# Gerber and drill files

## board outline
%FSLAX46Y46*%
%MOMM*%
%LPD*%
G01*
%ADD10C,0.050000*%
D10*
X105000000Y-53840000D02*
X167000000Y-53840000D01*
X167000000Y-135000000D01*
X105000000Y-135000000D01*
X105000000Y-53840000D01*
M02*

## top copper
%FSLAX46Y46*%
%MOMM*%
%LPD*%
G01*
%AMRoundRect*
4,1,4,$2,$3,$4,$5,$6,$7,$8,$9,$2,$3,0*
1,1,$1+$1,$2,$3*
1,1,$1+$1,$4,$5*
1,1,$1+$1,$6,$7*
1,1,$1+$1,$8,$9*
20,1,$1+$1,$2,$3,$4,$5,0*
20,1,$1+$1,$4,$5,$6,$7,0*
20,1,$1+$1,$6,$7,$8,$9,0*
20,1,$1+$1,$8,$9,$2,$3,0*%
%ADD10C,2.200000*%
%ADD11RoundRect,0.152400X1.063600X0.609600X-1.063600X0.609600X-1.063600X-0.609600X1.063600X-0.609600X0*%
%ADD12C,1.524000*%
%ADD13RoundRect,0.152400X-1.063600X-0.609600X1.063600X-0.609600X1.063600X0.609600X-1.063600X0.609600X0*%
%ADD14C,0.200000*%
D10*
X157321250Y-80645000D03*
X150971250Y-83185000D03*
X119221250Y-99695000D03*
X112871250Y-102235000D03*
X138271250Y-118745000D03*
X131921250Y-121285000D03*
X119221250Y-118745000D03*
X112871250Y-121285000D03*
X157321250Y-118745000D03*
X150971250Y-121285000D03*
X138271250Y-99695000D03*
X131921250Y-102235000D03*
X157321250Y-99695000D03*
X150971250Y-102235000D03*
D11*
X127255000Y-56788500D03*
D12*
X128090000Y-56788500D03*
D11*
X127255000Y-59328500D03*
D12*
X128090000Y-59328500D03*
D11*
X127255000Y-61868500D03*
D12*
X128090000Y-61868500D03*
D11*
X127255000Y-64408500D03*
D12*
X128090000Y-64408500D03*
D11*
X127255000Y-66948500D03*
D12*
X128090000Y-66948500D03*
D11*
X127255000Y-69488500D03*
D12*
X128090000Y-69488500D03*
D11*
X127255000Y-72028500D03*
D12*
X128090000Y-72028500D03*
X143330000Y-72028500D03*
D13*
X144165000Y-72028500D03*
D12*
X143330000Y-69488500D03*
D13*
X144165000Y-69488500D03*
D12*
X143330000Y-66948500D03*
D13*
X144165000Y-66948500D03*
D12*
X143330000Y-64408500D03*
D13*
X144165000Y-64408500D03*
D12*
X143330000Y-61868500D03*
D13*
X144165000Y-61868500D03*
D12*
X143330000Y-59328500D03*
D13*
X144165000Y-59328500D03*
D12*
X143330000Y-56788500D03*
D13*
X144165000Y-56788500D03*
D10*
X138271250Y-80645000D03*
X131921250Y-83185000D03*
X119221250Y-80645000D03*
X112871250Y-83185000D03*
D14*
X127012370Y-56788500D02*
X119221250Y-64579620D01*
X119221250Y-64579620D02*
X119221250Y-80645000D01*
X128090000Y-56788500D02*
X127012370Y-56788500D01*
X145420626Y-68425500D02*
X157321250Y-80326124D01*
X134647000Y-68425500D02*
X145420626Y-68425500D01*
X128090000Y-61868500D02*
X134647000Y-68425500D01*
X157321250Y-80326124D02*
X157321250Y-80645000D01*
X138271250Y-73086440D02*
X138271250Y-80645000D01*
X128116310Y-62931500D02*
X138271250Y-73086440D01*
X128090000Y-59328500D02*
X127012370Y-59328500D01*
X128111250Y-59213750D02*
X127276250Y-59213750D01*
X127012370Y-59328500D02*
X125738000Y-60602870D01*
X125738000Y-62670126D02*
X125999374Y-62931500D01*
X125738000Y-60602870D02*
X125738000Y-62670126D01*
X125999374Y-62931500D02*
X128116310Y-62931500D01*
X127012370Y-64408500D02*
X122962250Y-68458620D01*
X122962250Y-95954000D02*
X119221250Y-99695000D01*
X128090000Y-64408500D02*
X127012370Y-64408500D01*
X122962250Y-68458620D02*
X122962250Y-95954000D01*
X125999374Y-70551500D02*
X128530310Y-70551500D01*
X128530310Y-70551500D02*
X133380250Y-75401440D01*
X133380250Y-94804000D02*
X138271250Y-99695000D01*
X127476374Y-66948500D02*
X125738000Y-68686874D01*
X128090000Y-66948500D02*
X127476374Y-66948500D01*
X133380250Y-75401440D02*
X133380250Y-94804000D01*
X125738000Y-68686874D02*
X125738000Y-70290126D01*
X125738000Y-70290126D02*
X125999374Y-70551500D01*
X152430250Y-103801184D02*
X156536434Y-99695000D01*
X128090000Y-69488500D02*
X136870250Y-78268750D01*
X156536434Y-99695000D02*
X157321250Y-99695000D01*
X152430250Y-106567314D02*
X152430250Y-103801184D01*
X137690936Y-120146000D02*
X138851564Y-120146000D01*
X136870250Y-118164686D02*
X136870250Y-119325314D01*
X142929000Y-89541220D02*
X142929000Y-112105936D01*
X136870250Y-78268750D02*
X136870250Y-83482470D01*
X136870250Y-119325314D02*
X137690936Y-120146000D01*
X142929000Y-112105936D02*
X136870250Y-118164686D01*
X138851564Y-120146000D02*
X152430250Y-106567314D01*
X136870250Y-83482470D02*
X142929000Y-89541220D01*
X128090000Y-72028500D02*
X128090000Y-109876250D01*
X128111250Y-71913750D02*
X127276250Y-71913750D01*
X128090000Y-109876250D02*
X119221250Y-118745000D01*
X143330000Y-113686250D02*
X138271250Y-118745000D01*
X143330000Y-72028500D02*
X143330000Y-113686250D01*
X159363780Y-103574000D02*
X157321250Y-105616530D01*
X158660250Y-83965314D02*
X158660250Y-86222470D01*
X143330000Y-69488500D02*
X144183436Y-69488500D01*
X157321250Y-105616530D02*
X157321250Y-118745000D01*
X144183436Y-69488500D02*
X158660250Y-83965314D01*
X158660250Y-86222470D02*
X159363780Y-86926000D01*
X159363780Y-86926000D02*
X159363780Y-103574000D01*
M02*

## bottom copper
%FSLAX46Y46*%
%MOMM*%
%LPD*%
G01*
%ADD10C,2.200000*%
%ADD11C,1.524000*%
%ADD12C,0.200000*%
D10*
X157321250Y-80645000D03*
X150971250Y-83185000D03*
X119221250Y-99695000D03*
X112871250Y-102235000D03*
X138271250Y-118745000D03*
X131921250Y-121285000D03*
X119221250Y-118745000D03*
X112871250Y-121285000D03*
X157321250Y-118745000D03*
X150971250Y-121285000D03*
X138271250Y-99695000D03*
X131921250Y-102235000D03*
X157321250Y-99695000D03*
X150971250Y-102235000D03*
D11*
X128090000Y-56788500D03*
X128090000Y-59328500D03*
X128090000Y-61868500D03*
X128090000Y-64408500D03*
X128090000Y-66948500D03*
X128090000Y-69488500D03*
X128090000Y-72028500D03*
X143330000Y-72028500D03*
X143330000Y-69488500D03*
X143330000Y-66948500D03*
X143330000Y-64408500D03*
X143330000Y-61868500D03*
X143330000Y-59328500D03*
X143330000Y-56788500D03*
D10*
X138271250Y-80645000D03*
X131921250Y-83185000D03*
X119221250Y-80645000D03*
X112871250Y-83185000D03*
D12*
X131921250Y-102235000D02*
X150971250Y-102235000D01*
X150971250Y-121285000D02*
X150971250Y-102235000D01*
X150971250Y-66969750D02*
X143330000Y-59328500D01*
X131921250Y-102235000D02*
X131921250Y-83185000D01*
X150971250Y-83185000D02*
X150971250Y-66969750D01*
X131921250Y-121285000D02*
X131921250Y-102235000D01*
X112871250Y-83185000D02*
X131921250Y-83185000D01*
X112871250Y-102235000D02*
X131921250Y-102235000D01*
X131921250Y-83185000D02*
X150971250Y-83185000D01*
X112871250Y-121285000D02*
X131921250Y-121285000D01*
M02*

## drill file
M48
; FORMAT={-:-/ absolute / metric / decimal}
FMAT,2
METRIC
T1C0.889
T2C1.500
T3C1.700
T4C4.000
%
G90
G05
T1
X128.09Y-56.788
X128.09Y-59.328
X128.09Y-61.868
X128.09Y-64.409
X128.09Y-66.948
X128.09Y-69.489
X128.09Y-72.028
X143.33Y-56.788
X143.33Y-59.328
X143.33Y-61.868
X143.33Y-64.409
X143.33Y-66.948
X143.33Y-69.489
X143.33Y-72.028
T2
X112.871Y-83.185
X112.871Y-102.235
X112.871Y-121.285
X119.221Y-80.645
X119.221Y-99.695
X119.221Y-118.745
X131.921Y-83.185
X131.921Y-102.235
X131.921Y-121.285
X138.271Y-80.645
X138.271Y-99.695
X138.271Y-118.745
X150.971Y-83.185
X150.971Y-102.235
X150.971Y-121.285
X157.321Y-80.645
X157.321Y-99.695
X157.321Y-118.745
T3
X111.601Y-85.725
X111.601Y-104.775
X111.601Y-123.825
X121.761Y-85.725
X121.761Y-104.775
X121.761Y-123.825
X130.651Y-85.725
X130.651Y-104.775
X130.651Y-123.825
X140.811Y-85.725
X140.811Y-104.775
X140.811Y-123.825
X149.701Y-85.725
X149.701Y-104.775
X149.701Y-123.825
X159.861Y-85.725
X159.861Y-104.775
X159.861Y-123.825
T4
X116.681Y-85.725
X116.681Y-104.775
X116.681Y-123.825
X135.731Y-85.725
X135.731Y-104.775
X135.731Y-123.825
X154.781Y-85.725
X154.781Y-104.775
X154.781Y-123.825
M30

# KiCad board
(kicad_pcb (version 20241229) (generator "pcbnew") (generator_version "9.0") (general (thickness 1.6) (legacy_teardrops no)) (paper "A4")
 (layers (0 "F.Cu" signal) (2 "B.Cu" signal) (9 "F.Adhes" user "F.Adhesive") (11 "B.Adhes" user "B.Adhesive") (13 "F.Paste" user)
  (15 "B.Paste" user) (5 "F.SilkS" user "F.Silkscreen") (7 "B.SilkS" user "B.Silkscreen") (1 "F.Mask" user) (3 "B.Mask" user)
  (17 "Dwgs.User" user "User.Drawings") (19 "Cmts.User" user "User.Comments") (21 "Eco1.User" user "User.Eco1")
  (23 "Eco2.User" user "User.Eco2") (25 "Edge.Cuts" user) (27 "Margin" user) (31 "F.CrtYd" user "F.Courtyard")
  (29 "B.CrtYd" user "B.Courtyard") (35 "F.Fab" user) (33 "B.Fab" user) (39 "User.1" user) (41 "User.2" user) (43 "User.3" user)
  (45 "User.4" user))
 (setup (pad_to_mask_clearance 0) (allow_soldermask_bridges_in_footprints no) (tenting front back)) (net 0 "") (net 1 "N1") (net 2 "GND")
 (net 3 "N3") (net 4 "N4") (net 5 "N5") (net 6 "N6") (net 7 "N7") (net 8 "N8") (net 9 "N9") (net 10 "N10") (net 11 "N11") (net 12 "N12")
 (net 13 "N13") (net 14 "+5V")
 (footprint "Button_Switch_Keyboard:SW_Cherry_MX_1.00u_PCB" (layer "F.Cu") (at 157.32125 80.645)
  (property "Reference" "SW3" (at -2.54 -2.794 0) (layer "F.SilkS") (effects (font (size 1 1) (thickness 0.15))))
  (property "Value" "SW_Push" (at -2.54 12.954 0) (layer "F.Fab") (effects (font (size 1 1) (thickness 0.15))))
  (pad "" np_thru_hole circle (at -7.62 5.08) (size 1.7 1.7) (drill 1.7) (layers "*.Cu" "*.Mask"))
  (pad "" np_thru_hole circle (at -2.54 5.08) (size 4 4) (drill 4) (layers "*.Cu" "*.Mask"))
  (pad "" np_thru_hole circle (at 2.54 5.08) (size 1.7 1.7) (drill 1.7) (layers "*.Cu" "*.Mask"))
  (pad "1" thru_hole circle (at 0 0) (size 2.2 2.2) (drill 1.5) (layers "*.Cu" "*.Mask") (remove_unused_layers no) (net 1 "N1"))
  (pad "2" thru_hole circle (at -6.35 2.54) (size 2.2 2.2) (drill 1.5) (layers "*.Cu" "*.Mask") (remove_unused_layers no) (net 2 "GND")))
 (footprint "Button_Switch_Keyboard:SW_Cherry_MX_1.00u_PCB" (layer "F.Cu") (at 119.22125 99.695)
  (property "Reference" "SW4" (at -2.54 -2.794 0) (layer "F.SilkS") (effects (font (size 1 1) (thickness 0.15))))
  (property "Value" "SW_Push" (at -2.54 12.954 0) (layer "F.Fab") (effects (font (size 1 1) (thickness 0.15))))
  (pad "" np_thru_hole circle (at -7.62 5.08) (size 1.7 1.7) (drill 1.7) (layers "*.Cu" "*.Mask"))
  (pad "" np_thru_hole circle (at -2.54 5.08) (size 4 4) (drill 4) (layers "*.Cu" "*.Mask"))
  (pad "" np_thru_hole circle (at 2.54 5.08) (size 1.7 1.7) (drill 1.7) (layers "*.Cu" "*.Mask"))
  (pad "1" thru_hole circle (at 0 0) (size 2.2 2.2) (drill 1.5) (layers "*.Cu" "*.Mask") (remove_unused_layers no) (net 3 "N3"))
  (pad "2" thru_hole circle (at -6.35 2.54) (size 2.2 2.2) (drill 1.5) (layers "*.Cu" "*.Mask") (remove_unused_layers no) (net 2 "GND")))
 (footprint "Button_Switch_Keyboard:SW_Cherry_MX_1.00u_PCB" (layer "F.Cu") (at 138.27125 118.745)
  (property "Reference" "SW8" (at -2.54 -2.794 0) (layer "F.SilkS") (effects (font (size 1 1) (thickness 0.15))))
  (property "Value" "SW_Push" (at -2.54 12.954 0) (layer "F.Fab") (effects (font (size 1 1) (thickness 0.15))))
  (pad "" np_thru_hole circle (at -7.62 5.08) (size 1.7 1.7) (drill 1.7) (layers "*.Cu" "*.Mask"))
  (pad "" np_thru_hole circle (at -2.54 5.08) (size 4 4) (drill 4) (layers "*.Cu" "*.Mask"))
  (pad "" np_thru_hole circle (at 2.54 5.08) (size 1.7 1.7) (drill 1.7) (layers "*.Cu" "*.Mask"))
  (pad "1" thru_hole circle (at 0 0) (size 2.2 2.2) (drill 1.5) (layers "*.Cu" "*.Mask") (remove_unused_layers no) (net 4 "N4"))
  (pad "2" thru_hole circle (at -6.35 2.54) (size 2.2 2.2) (drill 1.5) (layers "*.Cu" "*.Mask") (remove_unused_layers no) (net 2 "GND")))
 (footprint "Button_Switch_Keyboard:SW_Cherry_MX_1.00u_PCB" (layer "F.Cu") (at 119.22125 118.745)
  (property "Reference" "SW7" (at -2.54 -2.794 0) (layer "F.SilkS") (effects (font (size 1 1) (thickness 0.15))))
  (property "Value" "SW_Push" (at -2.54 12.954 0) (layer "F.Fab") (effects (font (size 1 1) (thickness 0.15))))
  (pad "" np_thru_hole circle (at -7.62 5.08) (size 1.7 1.7) (drill 1.7) (layers "*.Cu" "*.Mask"))
  (pad "" np_thru_hole circle (at -2.54 5.08) (size 4 4) (drill 4) (layers "*.Cu" "*.Mask"))
  (pad "" np_thru_hole circle (at 2.54 5.08) (size 1.7 1.7) (drill 1.7) (layers "*.Cu" "*.Mask"))
  (pad "1" thru_hole circle (at 0 0) (size 2.2 2.2) (drill 1.5) (layers "*.Cu" "*.Mask") (remove_unused_layers no) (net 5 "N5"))
  (pad "2" thru_hole circle (at -6.35 2.54) (size 2.2 2.2) (drill 1.5) (layers "*.Cu" "*.Mask") (remove_unused_layers no) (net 2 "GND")))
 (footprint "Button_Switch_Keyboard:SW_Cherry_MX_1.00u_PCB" (layer "F.Cu") (at 157.32125 118.745)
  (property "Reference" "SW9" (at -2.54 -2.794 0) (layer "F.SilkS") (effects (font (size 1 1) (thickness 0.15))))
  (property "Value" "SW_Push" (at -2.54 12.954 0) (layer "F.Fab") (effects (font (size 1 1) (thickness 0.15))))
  (pad "" np_thru_hole circle (at -7.62 5.08) (size 1.7 1.7) (drill 1.7) (layers "*.Cu" "*.Mask"))
  (pad "" np_thru_hole circle (at -2.54 5.08) (size 4 4) (drill 4) (layers "*.Cu" "*.Mask"))
  (pad "" np_thru_hole circle (at 2.54 5.08) (size 1.7 1.7) (drill 1.7) (layers "*.Cu" "*.Mask"))
  (pad "1" thru_hole circle (at 0 0) (size 2.2 2.2) (drill 1.5) (layers "*.Cu" "*.Mask") (remove_unused_layers no) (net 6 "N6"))
  (pad "2" thru_hole circle (at -6.35 2.54) (size 2.2 2.2) (drill 1.5) (layers "*.Cu" "*.Mask") (remove_unused_layers no) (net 2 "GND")))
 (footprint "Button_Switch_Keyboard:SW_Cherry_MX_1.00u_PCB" (layer "F.Cu") (at 138.27125 99.695)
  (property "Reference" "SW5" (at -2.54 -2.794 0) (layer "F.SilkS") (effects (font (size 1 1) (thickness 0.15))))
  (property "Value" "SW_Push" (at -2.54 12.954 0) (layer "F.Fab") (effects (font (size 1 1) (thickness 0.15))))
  (pad "" np_thru_hole circle (at -7.62 5.08) (size 1.7 1.7) (drill 1.7) (layers "*.Cu" "*.Mask"))
  (pad "" np_thru_hole circle (at -2.54 5.08) (size 4 4) (drill 4) (layers "*.Cu" "*.Mask"))
  (pad "" np_thru_hole circle (at 2.54 5.08) (size 1.7 1.7) (drill 1.7) (layers "*.Cu" "*.Mask"))
  (pad "1" thru_hole circle (at 0 0) (size 2.2 2.2) (drill 1.5) (layers "*.Cu" "*.Mask") (remove_unused_layers no) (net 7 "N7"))
  (pad "2" thru_hole circle (at -6.35 2.54) (size 2.2 2.2) (drill 1.5) (layers "*.Cu" "*.Mask") (remove_unused_layers no) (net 2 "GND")))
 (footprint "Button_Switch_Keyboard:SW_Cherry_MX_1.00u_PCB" (layer "F.Cu") (at 157.32125 99.695)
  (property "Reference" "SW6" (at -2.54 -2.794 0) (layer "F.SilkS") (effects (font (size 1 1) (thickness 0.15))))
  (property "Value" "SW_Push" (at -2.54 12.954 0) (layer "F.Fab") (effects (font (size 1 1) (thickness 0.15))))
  (pad "" np_thru_hole circle (at -7.62 5.08) (size 1.7 1.7) (drill 1.7) (layers "*.Cu" "*.Mask"))
  (pad "" np_thru_hole circle (at -2.54 5.08) (size 4 4) (drill 4) (layers "*.Cu" "*.Mask"))
  (pad "" np_thru_hole circle (at 2.54 5.08) (size 1.7 1.7) (drill 1.7) (layers "*.Cu" "*.Mask"))
  (pad "1" thru_hole circle (at 0 0) (size 2.2 2.2) (drill 1.5) (layers "*.Cu" "*.Mask") (remove_unused_layers no) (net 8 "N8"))
  (pad "2" thru_hole circle (at -6.35 2.54) (size 2.2 2.2) (drill 1.5) (layers "*.Cu" "*.Mask") (remove_unused_layers no) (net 2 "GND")))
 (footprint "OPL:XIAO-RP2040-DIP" (layer "F.Cu") (at 135.71 64.4085)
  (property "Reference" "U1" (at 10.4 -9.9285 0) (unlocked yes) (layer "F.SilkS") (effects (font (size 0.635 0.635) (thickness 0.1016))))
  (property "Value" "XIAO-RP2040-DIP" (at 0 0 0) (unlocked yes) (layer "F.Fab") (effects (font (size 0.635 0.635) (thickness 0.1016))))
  (pad "1" smd roundrect (at -8.455 -7.62 180) (size 2.432 1.524) (layers "F.Cu" "F.Mask") (roundrect_rratio 0.1) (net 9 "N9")
   (thermal_bridge_angle 45))
  (pad "1" thru_hole circle (at -7.62 -7.62 180) (size 1.524 1.524) (drill 0.889) (layers "*.Cu" "*.Mask") (remove_unused_layers no)
   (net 9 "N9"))
  (pad "2" smd roundrect (at -8.455 -5.08 180) (size 2.432 1.524) (layers "F.Cu" "F.Mask") (roundrect_rratio 0.1) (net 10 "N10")
   (thermal_bridge_angle 45))
  (pad "2" thru_hole circle (at -7.62 -5.08 180) (size 1.524 1.524) (drill 0.889) (layers "*.Cu" "*.Mask") (remove_unused_layers no)
   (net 10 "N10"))
  (pad "3" smd roundrect (at -8.455 -2.54 180) (size 2.432 1.524) (layers "F.Cu" "F.Mask") (roundrect_rratio 0.1) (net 1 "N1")
   (thermal_bridge_angle 45))
  (pad "3" thru_hole circle (at -7.62 -2.54 180) (size 1.524 1.524) (drill 0.889) (layers "*.Cu" "*.Mask") (remove_unused_layers no)
   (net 1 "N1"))
  (pad "4" smd roundrect (at -8.455 0 180) (size 2.432 1.524) (layers "F.Cu" "F.Mask") (roundrect_rratio 0.1) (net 3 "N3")
   (thermal_bridge_angle 45))
  (pad "4" thru_hole circle (at -7.62 0 180) (size 1.524 1.524) (drill 0.889) (layers "*.Cu" "*.Mask") (remove_unused_layers no)
   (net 3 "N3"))
  (pad "5" smd roundrect (at -8.455 2.54 180) (size 2.432 1.524) (layers "F.Cu" "F.Mask") (roundrect_rratio 0.1) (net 7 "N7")
   (thermal_bridge_angle 45))
  (pad "5" thru_hole circle (at -7.62 2.54 180) (size 1.524 1.524) (drill 0.889) (layers "*.Cu" "*.Mask") (remove_unused_layers no)
   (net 7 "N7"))
  (pad "6" smd roundrect (at -8.455 5.08 180) (size 2.432 1.524) (layers "F.Cu" "F.Mask") (roundrect_rratio 0.1) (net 8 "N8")
   (thermal_bridge_angle 45))
  (pad "6" thru_hole circle (at -7.62 5.08 180) (size 1.524 1.524) (drill 0.889) (layers "*.Cu" "*.Mask") (remove_unused_layers no)
   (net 8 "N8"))
  (pad "7" smd roundrect (at -8.455 7.62 180) (size 2.432 1.524) (layers "F.Cu" "F.Mask") (roundrect_rratio 0.1) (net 5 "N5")
   (thermal_bridge_angle 45))
  (pad "7" thru_hole circle (at -7.62 7.62 180) (size 1.524 1.524) (drill 0.889) (layers "*.Cu" "*.Mask") (remove_unused_layers no)
   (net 5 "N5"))
  (pad "8" thru_hole circle (at 7.62 7.62) (size 1.524 1.524) (drill 0.889) (layers "*.Cu" "*.Mask") (remove_unused_layers no) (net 4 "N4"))
  (pad "8" smd roundrect (at 8.455 7.62) (size 2.432 1.524) (layers "F.Cu" "F.Mask") (roundrect_rratio 0.1) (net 4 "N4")
   (thermal_bridge_angle 45))
  (pad "9" thru_hole circle (at 7.62 5.08) (size 1.524 1.524) (drill 0.889) (layers "*.Cu" "*.Mask") (remove_unused_layers no) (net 6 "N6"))
  (pad "9" smd roundrect (at 8.455 5.08) (size 2.432 1.524) (layers "F.Cu" "F.Mask") (roundrect_rratio 0.1) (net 6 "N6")
   (thermal_bridge_angle 45))
  (pad "10" thru_hole circle (at 7.62 2.54) (size 1.524 1.524) (drill 0.889) (layers "*.Cu" "*.Mask") (remove_unused_layers no)
   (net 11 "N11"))
  (pad "10" smd roundrect (at 8.455 2.54) (size 2.432 1.524) (layers "F.Cu" "F.Mask") (roundrect_rratio 0.1) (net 11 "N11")
   (thermal_bridge_angle 45))
  (pad "11" thru_hole circle (at 7.62 0) (size 1.524 1.524) (drill 0.889) (layers "*.Cu" "*.Mask") (remove_unused_layers no) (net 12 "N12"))
  (pad "11" smd roundrect (at 8.455 0) (size 2.432 1.524) (layers "F.Cu" "F.Mask") (roundrect_rratio 0.1) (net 12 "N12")
   (thermal_bridge_angle 45))
  (pad "12" thru_hole circle (at 7.62 -2.54) (size 1.524 1.524) (drill 0.889) (layers "*.Cu" "*.Mask") (remove_unused_layers no)
   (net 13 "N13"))
  (pad "12" smd roundrect (at 8.455 -2.54) (size 2.432 1.524) (layers "F.Cu" "F.Mask") (roundrect_rratio 0.1) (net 13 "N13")
   (thermal_bridge_angle 45))
  (pad "13" thru_hole circle (at 7.62 -5.08) (size 1.524 1.524) (drill 0.889) (layers "*.Cu" "*.Mask") (remove_unused_layers no)
   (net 2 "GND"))
  (pad "13" smd roundrect (at 8.455 -5.08) (size 2.432 1.524) (layers "F.Cu" "F.Mask") (roundrect_rratio 0.1) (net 2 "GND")
   (thermal_bridge_angle 45))
  (pad "14" thru_hole circle (at 7.62 -7.62) (size 1.524 1.524) (drill 0.889) (layers "*.Cu" "*.Mask") (remove_unused_layers no)
   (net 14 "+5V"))
  (pad "14" smd roundrect (at 8.455 -7.62) (size 2.432 1.524) (layers "F.Cu" "F.Mask") (roundrect_rratio 0.1) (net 14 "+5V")
   (thermal_bridge_angle 45)))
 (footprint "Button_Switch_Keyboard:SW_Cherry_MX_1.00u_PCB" (layer "F.Cu") (at 138.27125 80.645)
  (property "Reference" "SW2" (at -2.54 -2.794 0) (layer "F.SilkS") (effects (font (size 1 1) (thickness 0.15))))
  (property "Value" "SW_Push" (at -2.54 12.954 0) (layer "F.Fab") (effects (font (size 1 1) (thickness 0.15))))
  (pad "" np_thru_hole circle (at -7.62 5.08) (size 1.7 1.7) (drill 1.7) (layers "*.Cu" "*.Mask"))
  (pad "" np_thru_hole circle (at -2.54 5.08) (size 4 4) (drill 4) (layers "*.Cu" "*.Mask"))
  (pad "" np_thru_hole circle (at 2.54 5.08) (size 1.7 1.7) (drill 1.7) (layers "*.Cu" "*.Mask"))
  (pad "1" thru_hole circle (at 0 0) (size 2.2 2.2) (drill 1.5) (layers "*.Cu" "*.Mask") (remove_unused_layers no) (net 10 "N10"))
  (pad "2" thru_hole circle (at -6.35 2.54) (size 2.2 2.2) (drill 1.5) (layers "*.Cu" "*.Mask") (remove_unused_layers no) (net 2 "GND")))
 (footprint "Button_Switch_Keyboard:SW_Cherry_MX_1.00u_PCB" (layer "F.Cu") (at 119.22125 80.645)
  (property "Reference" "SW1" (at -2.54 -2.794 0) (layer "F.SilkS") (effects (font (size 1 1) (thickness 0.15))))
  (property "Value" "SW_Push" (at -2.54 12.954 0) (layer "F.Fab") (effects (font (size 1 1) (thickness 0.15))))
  (pad "" np_thru_hole circle (at -7.62 5.08) (size 1.7 1.7) (drill 1.7) (layers "*.Cu" "*.Mask"))
  (pad "" np_thru_hole circle (at -2.54 5.08) (size 4 4) (drill 4) (layers "*.Cu" "*.Mask"))
  (pad "" np_thru_hole circle (at 2.54 5.08) (size 1.7 1.7) (drill 1.7) (layers "*.Cu" "*.Mask"))
  (pad "1" thru_hole circle (at 0 0) (size 2.2 2.2) (drill 1.5) (layers "*.Cu" "*.Mask") (remove_unused_layers no) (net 9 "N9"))
  (pad "2" thru_hole circle (at -6.35 2.54) (size 2.2 2.2) (drill 1.5) (layers "*.Cu" "*.Mask") (remove_unused_layers no) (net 2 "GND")))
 (gr_rect (start 105 53.84) (end 167 135) (stroke (width 0.05) (type default)) (fill no) (layer "Edge.Cuts"))
 (segment (start 127.01237 56.7885) (end 119.22125 64.57962) (width 0.2) (layer "F.Cu") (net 9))
 (segment (start 119.22125 64.57962) (end 119.22125 80.645) (width 0.2) (layer "F.Cu") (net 9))
 (segment (start 128.09 56.7885) (end 127.01237 56.7885) (width 0.2) (layer "F.Cu") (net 9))
 (segment (start 145.420626 68.4255) (end 157.32125 80.326124) (width 0.2) (layer "F.Cu") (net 1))
 (segment (start 134.647 68.4255) (end 145.420626 68.4255) (width 0.2) (layer "F.Cu") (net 1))
 (segment (start 128.09 61.8685) (end 134.647 68.4255) (width 0.2) (layer "F.Cu") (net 1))
 (segment (start 157.32125 80.326124) (end 157.32125 80.645) (width 0.2) (layer "F.Cu") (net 1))
 (segment (start 131.92125 102.235) (end 150.97125 102.235) (width 0.2) (layer "B.Cu") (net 2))
 (segment (start 150.97125 121.285) (end 150.97125 102.235) (width 0.2) (layer "B.Cu") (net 2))
 (segment (start 150.97125 66.96975) (end 143.33 59.3285) (width 0.2) (layer "B.Cu") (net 2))
 (segment (start 131.92125 102.235) (end 131.92125 83.185) (width 0.2) (layer "B.Cu") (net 2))
 (segment (start 150.97125 83.185) (end 150.97125 66.96975) (width 0.2) (layer "B.Cu") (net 2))
 (segment (start 131.92125 121.285) (end 131.92125 102.235) (width 0.2) (layer "B.Cu") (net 2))
 (segment (start 112.87125 83.185) (end 131.92125 83.185) (width 0.2) (layer "B.Cu") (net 2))
 (segment (start 112.87125 102.235) (end 131.92125 102.235) (width 0.2) (layer "B.Cu") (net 2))
 (segment (start 131.92125 83.185) (end 150.97125 83.185) (width 0.2) (layer "B.Cu") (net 2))
 (segment (start 112.87125 121.285) (end 131.92125 121.285) (width 0.2) (layer "B.Cu") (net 2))
 (segment (start 138.27125 73.08644) (end 138.27125 80.645) (width 0.2) (layer "F.Cu") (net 10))
 (segment (start 128.11631 62.9315) (end 138.27125 73.08644) (width 0.2) (layer "F.Cu") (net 10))
 (segment (start 128.09 59.3285) (end 127.01237 59.3285) (width 0.2) (layer "F.Cu") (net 10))
 (segment (start 128.11125 59.21375) (end 127.27625 59.21375) (width 0.2) (layer "F.Cu") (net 10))
 (segment (start 127.01237 59.3285) (end 125.738 60.60287) (width 0.2) (layer "F.Cu") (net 10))
 (segment (start 125.738 62.670126) (end 125.999374 62.9315) (width 0.2) (layer "F.Cu") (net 10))
 (segment (start 125.738 60.60287) (end 125.738 62.670126) (width 0.2) (layer "F.Cu") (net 10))
 (segment (start 125.999374 62.9315) (end 128.11631 62.9315) (width 0.2) (layer "F.Cu") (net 10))
 (segment (start 127.01237 64.4085) (end 122.96225 68.45862) (width 0.2) (layer "F.Cu") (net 3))
 (segment (start 122.96225 95.954) (end 119.22125 99.695) (width 0.2) (layer "F.Cu") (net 3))
 (segment (start 128.09 64.4085) (end 127.01237 64.4085) (width 0.2) (layer "F.Cu") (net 3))
 (segment (start 122.96225 68.45862) (end 122.96225 95.954) (width 0.2) (layer "F.Cu") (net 3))
 (segment (start 125.999374 70.5515) (end 128.53031 70.5515) (width 0.2) (layer "F.Cu") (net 7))
 (segment (start 128.53031 70.5515) (end 133.38025 75.40144) (width 0.2) (layer "F.Cu") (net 7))
 (segment (start 133.38025 94.804) (end 138.27125 99.695) (width 0.2) (layer "F.Cu") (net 7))
 (segment (start 127.476374 66.9485) (end 125.738 68.686874) (width 0.2) (layer "F.Cu") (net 7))
 (segment (start 128.09 66.9485) (end 127.476374 66.9485) (width 0.2) (layer "F.Cu") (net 7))
 (segment (start 133.38025 75.40144) (end 133.38025 94.804) (width 0.2) (layer "F.Cu") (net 7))
 (segment (start 125.738 68.686874) (end 125.738 70.290126) (width 0.2) (layer "F.Cu") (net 7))
 (segment (start 125.738 70.290126) (end 125.999374 70.5515) (width 0.2) (layer "F.Cu") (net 7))
 (segment (start 152.43025 103.801184) (end 156.536434 99.695) (width 0.2) (layer "F.Cu") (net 8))
 (segment (start 128.09 69.4885) (end 136.87025 78.26875) (width 0.2) (layer "F.Cu") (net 8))
 (segment (start 156.536434 99.695) (end 157.32125 99.695) (width 0.2) (layer "F.Cu") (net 8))
 (segment (start 152.43025 106.567314) (end 152.43025 103.801184) (width 0.2) (layer "F.Cu") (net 8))
 (segment (start 137.690936 120.146) (end 138.851564 120.146) (width 0.2) (layer "F.Cu") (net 8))
 (segment (start 136.87025 118.164686) (end 136.87025 119.325314) (width 0.2) (layer "F.Cu") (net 8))
 (segment (start 142.929 89.54122) (end 142.929 112.105936) (width 0.2) (layer "F.Cu") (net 8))
 (segment (start 136.87025 78.26875) (end 136.87025 83.48247) (width 0.2) (layer "F.Cu") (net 8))
 (segment (start 136.87025 119.325314) (end 137.690936 120.146) (width 0.2) (layer "F.Cu") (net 8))
 (segment (start 142.929 112.105936) (end 136.87025 118.164686) (width 0.2) (layer "F.Cu") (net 8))
 (segment (start 138.851564 120.146) (end 152.43025 106.567314) (width 0.2) (layer "F.Cu") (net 8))
 (segment (start 136.87025 83.48247) (end 142.929 89.54122) (width 0.2) (layer "F.Cu") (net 8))
 (segment (start 128.09 72.0285) (end 128.09 109.87625) (width 0.2) (layer "F.Cu") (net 5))
 (segment (start 128.11125 71.91375) (end 127.27625 71.91375) (width 0.2) (layer "F.Cu") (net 5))
 (segment (start 128.09 109.87625) (end 119.22125 118.745) (width 0.2) (layer "F.Cu") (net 5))
 (segment (start 143.33 113.68625) (end 138.27125 118.745) (width 0.2) (layer "F.Cu") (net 4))
 (segment (start 143.33 72.0285) (end 143.33 113.68625) (width 0.2) (layer "F.Cu") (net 4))
 (segment (start 159.36378 103.574) (end 157.32125 105.61653) (width 0.2) (layer "F.Cu") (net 6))
 (segment (start 158.66025 83.965314) (end 158.66025 86.22247) (width 0.2) (layer "F.Cu") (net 6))
 (segment (start 143.33 69.4885) (end 144.183436 69.4885) (width 0.2) (layer "F.Cu") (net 6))
 (segment (start 157.32125 105.61653) (end 157.32125 118.745) (width 0.2) (layer "F.Cu") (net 6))
 (segment (start 144.183436 69.4885) (end 158.66025 83.965314) (width 0.2) (layer "F.Cu") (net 6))
 (segment (start 158.66025 86.22247) (end 159.36378 86.926) (width 0.2) (layer "F.Cu") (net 6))
 (segment (start 159.36378 86.926) (end 159.36378 103.574) (width 0.2) (layer "F.Cu") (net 6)))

